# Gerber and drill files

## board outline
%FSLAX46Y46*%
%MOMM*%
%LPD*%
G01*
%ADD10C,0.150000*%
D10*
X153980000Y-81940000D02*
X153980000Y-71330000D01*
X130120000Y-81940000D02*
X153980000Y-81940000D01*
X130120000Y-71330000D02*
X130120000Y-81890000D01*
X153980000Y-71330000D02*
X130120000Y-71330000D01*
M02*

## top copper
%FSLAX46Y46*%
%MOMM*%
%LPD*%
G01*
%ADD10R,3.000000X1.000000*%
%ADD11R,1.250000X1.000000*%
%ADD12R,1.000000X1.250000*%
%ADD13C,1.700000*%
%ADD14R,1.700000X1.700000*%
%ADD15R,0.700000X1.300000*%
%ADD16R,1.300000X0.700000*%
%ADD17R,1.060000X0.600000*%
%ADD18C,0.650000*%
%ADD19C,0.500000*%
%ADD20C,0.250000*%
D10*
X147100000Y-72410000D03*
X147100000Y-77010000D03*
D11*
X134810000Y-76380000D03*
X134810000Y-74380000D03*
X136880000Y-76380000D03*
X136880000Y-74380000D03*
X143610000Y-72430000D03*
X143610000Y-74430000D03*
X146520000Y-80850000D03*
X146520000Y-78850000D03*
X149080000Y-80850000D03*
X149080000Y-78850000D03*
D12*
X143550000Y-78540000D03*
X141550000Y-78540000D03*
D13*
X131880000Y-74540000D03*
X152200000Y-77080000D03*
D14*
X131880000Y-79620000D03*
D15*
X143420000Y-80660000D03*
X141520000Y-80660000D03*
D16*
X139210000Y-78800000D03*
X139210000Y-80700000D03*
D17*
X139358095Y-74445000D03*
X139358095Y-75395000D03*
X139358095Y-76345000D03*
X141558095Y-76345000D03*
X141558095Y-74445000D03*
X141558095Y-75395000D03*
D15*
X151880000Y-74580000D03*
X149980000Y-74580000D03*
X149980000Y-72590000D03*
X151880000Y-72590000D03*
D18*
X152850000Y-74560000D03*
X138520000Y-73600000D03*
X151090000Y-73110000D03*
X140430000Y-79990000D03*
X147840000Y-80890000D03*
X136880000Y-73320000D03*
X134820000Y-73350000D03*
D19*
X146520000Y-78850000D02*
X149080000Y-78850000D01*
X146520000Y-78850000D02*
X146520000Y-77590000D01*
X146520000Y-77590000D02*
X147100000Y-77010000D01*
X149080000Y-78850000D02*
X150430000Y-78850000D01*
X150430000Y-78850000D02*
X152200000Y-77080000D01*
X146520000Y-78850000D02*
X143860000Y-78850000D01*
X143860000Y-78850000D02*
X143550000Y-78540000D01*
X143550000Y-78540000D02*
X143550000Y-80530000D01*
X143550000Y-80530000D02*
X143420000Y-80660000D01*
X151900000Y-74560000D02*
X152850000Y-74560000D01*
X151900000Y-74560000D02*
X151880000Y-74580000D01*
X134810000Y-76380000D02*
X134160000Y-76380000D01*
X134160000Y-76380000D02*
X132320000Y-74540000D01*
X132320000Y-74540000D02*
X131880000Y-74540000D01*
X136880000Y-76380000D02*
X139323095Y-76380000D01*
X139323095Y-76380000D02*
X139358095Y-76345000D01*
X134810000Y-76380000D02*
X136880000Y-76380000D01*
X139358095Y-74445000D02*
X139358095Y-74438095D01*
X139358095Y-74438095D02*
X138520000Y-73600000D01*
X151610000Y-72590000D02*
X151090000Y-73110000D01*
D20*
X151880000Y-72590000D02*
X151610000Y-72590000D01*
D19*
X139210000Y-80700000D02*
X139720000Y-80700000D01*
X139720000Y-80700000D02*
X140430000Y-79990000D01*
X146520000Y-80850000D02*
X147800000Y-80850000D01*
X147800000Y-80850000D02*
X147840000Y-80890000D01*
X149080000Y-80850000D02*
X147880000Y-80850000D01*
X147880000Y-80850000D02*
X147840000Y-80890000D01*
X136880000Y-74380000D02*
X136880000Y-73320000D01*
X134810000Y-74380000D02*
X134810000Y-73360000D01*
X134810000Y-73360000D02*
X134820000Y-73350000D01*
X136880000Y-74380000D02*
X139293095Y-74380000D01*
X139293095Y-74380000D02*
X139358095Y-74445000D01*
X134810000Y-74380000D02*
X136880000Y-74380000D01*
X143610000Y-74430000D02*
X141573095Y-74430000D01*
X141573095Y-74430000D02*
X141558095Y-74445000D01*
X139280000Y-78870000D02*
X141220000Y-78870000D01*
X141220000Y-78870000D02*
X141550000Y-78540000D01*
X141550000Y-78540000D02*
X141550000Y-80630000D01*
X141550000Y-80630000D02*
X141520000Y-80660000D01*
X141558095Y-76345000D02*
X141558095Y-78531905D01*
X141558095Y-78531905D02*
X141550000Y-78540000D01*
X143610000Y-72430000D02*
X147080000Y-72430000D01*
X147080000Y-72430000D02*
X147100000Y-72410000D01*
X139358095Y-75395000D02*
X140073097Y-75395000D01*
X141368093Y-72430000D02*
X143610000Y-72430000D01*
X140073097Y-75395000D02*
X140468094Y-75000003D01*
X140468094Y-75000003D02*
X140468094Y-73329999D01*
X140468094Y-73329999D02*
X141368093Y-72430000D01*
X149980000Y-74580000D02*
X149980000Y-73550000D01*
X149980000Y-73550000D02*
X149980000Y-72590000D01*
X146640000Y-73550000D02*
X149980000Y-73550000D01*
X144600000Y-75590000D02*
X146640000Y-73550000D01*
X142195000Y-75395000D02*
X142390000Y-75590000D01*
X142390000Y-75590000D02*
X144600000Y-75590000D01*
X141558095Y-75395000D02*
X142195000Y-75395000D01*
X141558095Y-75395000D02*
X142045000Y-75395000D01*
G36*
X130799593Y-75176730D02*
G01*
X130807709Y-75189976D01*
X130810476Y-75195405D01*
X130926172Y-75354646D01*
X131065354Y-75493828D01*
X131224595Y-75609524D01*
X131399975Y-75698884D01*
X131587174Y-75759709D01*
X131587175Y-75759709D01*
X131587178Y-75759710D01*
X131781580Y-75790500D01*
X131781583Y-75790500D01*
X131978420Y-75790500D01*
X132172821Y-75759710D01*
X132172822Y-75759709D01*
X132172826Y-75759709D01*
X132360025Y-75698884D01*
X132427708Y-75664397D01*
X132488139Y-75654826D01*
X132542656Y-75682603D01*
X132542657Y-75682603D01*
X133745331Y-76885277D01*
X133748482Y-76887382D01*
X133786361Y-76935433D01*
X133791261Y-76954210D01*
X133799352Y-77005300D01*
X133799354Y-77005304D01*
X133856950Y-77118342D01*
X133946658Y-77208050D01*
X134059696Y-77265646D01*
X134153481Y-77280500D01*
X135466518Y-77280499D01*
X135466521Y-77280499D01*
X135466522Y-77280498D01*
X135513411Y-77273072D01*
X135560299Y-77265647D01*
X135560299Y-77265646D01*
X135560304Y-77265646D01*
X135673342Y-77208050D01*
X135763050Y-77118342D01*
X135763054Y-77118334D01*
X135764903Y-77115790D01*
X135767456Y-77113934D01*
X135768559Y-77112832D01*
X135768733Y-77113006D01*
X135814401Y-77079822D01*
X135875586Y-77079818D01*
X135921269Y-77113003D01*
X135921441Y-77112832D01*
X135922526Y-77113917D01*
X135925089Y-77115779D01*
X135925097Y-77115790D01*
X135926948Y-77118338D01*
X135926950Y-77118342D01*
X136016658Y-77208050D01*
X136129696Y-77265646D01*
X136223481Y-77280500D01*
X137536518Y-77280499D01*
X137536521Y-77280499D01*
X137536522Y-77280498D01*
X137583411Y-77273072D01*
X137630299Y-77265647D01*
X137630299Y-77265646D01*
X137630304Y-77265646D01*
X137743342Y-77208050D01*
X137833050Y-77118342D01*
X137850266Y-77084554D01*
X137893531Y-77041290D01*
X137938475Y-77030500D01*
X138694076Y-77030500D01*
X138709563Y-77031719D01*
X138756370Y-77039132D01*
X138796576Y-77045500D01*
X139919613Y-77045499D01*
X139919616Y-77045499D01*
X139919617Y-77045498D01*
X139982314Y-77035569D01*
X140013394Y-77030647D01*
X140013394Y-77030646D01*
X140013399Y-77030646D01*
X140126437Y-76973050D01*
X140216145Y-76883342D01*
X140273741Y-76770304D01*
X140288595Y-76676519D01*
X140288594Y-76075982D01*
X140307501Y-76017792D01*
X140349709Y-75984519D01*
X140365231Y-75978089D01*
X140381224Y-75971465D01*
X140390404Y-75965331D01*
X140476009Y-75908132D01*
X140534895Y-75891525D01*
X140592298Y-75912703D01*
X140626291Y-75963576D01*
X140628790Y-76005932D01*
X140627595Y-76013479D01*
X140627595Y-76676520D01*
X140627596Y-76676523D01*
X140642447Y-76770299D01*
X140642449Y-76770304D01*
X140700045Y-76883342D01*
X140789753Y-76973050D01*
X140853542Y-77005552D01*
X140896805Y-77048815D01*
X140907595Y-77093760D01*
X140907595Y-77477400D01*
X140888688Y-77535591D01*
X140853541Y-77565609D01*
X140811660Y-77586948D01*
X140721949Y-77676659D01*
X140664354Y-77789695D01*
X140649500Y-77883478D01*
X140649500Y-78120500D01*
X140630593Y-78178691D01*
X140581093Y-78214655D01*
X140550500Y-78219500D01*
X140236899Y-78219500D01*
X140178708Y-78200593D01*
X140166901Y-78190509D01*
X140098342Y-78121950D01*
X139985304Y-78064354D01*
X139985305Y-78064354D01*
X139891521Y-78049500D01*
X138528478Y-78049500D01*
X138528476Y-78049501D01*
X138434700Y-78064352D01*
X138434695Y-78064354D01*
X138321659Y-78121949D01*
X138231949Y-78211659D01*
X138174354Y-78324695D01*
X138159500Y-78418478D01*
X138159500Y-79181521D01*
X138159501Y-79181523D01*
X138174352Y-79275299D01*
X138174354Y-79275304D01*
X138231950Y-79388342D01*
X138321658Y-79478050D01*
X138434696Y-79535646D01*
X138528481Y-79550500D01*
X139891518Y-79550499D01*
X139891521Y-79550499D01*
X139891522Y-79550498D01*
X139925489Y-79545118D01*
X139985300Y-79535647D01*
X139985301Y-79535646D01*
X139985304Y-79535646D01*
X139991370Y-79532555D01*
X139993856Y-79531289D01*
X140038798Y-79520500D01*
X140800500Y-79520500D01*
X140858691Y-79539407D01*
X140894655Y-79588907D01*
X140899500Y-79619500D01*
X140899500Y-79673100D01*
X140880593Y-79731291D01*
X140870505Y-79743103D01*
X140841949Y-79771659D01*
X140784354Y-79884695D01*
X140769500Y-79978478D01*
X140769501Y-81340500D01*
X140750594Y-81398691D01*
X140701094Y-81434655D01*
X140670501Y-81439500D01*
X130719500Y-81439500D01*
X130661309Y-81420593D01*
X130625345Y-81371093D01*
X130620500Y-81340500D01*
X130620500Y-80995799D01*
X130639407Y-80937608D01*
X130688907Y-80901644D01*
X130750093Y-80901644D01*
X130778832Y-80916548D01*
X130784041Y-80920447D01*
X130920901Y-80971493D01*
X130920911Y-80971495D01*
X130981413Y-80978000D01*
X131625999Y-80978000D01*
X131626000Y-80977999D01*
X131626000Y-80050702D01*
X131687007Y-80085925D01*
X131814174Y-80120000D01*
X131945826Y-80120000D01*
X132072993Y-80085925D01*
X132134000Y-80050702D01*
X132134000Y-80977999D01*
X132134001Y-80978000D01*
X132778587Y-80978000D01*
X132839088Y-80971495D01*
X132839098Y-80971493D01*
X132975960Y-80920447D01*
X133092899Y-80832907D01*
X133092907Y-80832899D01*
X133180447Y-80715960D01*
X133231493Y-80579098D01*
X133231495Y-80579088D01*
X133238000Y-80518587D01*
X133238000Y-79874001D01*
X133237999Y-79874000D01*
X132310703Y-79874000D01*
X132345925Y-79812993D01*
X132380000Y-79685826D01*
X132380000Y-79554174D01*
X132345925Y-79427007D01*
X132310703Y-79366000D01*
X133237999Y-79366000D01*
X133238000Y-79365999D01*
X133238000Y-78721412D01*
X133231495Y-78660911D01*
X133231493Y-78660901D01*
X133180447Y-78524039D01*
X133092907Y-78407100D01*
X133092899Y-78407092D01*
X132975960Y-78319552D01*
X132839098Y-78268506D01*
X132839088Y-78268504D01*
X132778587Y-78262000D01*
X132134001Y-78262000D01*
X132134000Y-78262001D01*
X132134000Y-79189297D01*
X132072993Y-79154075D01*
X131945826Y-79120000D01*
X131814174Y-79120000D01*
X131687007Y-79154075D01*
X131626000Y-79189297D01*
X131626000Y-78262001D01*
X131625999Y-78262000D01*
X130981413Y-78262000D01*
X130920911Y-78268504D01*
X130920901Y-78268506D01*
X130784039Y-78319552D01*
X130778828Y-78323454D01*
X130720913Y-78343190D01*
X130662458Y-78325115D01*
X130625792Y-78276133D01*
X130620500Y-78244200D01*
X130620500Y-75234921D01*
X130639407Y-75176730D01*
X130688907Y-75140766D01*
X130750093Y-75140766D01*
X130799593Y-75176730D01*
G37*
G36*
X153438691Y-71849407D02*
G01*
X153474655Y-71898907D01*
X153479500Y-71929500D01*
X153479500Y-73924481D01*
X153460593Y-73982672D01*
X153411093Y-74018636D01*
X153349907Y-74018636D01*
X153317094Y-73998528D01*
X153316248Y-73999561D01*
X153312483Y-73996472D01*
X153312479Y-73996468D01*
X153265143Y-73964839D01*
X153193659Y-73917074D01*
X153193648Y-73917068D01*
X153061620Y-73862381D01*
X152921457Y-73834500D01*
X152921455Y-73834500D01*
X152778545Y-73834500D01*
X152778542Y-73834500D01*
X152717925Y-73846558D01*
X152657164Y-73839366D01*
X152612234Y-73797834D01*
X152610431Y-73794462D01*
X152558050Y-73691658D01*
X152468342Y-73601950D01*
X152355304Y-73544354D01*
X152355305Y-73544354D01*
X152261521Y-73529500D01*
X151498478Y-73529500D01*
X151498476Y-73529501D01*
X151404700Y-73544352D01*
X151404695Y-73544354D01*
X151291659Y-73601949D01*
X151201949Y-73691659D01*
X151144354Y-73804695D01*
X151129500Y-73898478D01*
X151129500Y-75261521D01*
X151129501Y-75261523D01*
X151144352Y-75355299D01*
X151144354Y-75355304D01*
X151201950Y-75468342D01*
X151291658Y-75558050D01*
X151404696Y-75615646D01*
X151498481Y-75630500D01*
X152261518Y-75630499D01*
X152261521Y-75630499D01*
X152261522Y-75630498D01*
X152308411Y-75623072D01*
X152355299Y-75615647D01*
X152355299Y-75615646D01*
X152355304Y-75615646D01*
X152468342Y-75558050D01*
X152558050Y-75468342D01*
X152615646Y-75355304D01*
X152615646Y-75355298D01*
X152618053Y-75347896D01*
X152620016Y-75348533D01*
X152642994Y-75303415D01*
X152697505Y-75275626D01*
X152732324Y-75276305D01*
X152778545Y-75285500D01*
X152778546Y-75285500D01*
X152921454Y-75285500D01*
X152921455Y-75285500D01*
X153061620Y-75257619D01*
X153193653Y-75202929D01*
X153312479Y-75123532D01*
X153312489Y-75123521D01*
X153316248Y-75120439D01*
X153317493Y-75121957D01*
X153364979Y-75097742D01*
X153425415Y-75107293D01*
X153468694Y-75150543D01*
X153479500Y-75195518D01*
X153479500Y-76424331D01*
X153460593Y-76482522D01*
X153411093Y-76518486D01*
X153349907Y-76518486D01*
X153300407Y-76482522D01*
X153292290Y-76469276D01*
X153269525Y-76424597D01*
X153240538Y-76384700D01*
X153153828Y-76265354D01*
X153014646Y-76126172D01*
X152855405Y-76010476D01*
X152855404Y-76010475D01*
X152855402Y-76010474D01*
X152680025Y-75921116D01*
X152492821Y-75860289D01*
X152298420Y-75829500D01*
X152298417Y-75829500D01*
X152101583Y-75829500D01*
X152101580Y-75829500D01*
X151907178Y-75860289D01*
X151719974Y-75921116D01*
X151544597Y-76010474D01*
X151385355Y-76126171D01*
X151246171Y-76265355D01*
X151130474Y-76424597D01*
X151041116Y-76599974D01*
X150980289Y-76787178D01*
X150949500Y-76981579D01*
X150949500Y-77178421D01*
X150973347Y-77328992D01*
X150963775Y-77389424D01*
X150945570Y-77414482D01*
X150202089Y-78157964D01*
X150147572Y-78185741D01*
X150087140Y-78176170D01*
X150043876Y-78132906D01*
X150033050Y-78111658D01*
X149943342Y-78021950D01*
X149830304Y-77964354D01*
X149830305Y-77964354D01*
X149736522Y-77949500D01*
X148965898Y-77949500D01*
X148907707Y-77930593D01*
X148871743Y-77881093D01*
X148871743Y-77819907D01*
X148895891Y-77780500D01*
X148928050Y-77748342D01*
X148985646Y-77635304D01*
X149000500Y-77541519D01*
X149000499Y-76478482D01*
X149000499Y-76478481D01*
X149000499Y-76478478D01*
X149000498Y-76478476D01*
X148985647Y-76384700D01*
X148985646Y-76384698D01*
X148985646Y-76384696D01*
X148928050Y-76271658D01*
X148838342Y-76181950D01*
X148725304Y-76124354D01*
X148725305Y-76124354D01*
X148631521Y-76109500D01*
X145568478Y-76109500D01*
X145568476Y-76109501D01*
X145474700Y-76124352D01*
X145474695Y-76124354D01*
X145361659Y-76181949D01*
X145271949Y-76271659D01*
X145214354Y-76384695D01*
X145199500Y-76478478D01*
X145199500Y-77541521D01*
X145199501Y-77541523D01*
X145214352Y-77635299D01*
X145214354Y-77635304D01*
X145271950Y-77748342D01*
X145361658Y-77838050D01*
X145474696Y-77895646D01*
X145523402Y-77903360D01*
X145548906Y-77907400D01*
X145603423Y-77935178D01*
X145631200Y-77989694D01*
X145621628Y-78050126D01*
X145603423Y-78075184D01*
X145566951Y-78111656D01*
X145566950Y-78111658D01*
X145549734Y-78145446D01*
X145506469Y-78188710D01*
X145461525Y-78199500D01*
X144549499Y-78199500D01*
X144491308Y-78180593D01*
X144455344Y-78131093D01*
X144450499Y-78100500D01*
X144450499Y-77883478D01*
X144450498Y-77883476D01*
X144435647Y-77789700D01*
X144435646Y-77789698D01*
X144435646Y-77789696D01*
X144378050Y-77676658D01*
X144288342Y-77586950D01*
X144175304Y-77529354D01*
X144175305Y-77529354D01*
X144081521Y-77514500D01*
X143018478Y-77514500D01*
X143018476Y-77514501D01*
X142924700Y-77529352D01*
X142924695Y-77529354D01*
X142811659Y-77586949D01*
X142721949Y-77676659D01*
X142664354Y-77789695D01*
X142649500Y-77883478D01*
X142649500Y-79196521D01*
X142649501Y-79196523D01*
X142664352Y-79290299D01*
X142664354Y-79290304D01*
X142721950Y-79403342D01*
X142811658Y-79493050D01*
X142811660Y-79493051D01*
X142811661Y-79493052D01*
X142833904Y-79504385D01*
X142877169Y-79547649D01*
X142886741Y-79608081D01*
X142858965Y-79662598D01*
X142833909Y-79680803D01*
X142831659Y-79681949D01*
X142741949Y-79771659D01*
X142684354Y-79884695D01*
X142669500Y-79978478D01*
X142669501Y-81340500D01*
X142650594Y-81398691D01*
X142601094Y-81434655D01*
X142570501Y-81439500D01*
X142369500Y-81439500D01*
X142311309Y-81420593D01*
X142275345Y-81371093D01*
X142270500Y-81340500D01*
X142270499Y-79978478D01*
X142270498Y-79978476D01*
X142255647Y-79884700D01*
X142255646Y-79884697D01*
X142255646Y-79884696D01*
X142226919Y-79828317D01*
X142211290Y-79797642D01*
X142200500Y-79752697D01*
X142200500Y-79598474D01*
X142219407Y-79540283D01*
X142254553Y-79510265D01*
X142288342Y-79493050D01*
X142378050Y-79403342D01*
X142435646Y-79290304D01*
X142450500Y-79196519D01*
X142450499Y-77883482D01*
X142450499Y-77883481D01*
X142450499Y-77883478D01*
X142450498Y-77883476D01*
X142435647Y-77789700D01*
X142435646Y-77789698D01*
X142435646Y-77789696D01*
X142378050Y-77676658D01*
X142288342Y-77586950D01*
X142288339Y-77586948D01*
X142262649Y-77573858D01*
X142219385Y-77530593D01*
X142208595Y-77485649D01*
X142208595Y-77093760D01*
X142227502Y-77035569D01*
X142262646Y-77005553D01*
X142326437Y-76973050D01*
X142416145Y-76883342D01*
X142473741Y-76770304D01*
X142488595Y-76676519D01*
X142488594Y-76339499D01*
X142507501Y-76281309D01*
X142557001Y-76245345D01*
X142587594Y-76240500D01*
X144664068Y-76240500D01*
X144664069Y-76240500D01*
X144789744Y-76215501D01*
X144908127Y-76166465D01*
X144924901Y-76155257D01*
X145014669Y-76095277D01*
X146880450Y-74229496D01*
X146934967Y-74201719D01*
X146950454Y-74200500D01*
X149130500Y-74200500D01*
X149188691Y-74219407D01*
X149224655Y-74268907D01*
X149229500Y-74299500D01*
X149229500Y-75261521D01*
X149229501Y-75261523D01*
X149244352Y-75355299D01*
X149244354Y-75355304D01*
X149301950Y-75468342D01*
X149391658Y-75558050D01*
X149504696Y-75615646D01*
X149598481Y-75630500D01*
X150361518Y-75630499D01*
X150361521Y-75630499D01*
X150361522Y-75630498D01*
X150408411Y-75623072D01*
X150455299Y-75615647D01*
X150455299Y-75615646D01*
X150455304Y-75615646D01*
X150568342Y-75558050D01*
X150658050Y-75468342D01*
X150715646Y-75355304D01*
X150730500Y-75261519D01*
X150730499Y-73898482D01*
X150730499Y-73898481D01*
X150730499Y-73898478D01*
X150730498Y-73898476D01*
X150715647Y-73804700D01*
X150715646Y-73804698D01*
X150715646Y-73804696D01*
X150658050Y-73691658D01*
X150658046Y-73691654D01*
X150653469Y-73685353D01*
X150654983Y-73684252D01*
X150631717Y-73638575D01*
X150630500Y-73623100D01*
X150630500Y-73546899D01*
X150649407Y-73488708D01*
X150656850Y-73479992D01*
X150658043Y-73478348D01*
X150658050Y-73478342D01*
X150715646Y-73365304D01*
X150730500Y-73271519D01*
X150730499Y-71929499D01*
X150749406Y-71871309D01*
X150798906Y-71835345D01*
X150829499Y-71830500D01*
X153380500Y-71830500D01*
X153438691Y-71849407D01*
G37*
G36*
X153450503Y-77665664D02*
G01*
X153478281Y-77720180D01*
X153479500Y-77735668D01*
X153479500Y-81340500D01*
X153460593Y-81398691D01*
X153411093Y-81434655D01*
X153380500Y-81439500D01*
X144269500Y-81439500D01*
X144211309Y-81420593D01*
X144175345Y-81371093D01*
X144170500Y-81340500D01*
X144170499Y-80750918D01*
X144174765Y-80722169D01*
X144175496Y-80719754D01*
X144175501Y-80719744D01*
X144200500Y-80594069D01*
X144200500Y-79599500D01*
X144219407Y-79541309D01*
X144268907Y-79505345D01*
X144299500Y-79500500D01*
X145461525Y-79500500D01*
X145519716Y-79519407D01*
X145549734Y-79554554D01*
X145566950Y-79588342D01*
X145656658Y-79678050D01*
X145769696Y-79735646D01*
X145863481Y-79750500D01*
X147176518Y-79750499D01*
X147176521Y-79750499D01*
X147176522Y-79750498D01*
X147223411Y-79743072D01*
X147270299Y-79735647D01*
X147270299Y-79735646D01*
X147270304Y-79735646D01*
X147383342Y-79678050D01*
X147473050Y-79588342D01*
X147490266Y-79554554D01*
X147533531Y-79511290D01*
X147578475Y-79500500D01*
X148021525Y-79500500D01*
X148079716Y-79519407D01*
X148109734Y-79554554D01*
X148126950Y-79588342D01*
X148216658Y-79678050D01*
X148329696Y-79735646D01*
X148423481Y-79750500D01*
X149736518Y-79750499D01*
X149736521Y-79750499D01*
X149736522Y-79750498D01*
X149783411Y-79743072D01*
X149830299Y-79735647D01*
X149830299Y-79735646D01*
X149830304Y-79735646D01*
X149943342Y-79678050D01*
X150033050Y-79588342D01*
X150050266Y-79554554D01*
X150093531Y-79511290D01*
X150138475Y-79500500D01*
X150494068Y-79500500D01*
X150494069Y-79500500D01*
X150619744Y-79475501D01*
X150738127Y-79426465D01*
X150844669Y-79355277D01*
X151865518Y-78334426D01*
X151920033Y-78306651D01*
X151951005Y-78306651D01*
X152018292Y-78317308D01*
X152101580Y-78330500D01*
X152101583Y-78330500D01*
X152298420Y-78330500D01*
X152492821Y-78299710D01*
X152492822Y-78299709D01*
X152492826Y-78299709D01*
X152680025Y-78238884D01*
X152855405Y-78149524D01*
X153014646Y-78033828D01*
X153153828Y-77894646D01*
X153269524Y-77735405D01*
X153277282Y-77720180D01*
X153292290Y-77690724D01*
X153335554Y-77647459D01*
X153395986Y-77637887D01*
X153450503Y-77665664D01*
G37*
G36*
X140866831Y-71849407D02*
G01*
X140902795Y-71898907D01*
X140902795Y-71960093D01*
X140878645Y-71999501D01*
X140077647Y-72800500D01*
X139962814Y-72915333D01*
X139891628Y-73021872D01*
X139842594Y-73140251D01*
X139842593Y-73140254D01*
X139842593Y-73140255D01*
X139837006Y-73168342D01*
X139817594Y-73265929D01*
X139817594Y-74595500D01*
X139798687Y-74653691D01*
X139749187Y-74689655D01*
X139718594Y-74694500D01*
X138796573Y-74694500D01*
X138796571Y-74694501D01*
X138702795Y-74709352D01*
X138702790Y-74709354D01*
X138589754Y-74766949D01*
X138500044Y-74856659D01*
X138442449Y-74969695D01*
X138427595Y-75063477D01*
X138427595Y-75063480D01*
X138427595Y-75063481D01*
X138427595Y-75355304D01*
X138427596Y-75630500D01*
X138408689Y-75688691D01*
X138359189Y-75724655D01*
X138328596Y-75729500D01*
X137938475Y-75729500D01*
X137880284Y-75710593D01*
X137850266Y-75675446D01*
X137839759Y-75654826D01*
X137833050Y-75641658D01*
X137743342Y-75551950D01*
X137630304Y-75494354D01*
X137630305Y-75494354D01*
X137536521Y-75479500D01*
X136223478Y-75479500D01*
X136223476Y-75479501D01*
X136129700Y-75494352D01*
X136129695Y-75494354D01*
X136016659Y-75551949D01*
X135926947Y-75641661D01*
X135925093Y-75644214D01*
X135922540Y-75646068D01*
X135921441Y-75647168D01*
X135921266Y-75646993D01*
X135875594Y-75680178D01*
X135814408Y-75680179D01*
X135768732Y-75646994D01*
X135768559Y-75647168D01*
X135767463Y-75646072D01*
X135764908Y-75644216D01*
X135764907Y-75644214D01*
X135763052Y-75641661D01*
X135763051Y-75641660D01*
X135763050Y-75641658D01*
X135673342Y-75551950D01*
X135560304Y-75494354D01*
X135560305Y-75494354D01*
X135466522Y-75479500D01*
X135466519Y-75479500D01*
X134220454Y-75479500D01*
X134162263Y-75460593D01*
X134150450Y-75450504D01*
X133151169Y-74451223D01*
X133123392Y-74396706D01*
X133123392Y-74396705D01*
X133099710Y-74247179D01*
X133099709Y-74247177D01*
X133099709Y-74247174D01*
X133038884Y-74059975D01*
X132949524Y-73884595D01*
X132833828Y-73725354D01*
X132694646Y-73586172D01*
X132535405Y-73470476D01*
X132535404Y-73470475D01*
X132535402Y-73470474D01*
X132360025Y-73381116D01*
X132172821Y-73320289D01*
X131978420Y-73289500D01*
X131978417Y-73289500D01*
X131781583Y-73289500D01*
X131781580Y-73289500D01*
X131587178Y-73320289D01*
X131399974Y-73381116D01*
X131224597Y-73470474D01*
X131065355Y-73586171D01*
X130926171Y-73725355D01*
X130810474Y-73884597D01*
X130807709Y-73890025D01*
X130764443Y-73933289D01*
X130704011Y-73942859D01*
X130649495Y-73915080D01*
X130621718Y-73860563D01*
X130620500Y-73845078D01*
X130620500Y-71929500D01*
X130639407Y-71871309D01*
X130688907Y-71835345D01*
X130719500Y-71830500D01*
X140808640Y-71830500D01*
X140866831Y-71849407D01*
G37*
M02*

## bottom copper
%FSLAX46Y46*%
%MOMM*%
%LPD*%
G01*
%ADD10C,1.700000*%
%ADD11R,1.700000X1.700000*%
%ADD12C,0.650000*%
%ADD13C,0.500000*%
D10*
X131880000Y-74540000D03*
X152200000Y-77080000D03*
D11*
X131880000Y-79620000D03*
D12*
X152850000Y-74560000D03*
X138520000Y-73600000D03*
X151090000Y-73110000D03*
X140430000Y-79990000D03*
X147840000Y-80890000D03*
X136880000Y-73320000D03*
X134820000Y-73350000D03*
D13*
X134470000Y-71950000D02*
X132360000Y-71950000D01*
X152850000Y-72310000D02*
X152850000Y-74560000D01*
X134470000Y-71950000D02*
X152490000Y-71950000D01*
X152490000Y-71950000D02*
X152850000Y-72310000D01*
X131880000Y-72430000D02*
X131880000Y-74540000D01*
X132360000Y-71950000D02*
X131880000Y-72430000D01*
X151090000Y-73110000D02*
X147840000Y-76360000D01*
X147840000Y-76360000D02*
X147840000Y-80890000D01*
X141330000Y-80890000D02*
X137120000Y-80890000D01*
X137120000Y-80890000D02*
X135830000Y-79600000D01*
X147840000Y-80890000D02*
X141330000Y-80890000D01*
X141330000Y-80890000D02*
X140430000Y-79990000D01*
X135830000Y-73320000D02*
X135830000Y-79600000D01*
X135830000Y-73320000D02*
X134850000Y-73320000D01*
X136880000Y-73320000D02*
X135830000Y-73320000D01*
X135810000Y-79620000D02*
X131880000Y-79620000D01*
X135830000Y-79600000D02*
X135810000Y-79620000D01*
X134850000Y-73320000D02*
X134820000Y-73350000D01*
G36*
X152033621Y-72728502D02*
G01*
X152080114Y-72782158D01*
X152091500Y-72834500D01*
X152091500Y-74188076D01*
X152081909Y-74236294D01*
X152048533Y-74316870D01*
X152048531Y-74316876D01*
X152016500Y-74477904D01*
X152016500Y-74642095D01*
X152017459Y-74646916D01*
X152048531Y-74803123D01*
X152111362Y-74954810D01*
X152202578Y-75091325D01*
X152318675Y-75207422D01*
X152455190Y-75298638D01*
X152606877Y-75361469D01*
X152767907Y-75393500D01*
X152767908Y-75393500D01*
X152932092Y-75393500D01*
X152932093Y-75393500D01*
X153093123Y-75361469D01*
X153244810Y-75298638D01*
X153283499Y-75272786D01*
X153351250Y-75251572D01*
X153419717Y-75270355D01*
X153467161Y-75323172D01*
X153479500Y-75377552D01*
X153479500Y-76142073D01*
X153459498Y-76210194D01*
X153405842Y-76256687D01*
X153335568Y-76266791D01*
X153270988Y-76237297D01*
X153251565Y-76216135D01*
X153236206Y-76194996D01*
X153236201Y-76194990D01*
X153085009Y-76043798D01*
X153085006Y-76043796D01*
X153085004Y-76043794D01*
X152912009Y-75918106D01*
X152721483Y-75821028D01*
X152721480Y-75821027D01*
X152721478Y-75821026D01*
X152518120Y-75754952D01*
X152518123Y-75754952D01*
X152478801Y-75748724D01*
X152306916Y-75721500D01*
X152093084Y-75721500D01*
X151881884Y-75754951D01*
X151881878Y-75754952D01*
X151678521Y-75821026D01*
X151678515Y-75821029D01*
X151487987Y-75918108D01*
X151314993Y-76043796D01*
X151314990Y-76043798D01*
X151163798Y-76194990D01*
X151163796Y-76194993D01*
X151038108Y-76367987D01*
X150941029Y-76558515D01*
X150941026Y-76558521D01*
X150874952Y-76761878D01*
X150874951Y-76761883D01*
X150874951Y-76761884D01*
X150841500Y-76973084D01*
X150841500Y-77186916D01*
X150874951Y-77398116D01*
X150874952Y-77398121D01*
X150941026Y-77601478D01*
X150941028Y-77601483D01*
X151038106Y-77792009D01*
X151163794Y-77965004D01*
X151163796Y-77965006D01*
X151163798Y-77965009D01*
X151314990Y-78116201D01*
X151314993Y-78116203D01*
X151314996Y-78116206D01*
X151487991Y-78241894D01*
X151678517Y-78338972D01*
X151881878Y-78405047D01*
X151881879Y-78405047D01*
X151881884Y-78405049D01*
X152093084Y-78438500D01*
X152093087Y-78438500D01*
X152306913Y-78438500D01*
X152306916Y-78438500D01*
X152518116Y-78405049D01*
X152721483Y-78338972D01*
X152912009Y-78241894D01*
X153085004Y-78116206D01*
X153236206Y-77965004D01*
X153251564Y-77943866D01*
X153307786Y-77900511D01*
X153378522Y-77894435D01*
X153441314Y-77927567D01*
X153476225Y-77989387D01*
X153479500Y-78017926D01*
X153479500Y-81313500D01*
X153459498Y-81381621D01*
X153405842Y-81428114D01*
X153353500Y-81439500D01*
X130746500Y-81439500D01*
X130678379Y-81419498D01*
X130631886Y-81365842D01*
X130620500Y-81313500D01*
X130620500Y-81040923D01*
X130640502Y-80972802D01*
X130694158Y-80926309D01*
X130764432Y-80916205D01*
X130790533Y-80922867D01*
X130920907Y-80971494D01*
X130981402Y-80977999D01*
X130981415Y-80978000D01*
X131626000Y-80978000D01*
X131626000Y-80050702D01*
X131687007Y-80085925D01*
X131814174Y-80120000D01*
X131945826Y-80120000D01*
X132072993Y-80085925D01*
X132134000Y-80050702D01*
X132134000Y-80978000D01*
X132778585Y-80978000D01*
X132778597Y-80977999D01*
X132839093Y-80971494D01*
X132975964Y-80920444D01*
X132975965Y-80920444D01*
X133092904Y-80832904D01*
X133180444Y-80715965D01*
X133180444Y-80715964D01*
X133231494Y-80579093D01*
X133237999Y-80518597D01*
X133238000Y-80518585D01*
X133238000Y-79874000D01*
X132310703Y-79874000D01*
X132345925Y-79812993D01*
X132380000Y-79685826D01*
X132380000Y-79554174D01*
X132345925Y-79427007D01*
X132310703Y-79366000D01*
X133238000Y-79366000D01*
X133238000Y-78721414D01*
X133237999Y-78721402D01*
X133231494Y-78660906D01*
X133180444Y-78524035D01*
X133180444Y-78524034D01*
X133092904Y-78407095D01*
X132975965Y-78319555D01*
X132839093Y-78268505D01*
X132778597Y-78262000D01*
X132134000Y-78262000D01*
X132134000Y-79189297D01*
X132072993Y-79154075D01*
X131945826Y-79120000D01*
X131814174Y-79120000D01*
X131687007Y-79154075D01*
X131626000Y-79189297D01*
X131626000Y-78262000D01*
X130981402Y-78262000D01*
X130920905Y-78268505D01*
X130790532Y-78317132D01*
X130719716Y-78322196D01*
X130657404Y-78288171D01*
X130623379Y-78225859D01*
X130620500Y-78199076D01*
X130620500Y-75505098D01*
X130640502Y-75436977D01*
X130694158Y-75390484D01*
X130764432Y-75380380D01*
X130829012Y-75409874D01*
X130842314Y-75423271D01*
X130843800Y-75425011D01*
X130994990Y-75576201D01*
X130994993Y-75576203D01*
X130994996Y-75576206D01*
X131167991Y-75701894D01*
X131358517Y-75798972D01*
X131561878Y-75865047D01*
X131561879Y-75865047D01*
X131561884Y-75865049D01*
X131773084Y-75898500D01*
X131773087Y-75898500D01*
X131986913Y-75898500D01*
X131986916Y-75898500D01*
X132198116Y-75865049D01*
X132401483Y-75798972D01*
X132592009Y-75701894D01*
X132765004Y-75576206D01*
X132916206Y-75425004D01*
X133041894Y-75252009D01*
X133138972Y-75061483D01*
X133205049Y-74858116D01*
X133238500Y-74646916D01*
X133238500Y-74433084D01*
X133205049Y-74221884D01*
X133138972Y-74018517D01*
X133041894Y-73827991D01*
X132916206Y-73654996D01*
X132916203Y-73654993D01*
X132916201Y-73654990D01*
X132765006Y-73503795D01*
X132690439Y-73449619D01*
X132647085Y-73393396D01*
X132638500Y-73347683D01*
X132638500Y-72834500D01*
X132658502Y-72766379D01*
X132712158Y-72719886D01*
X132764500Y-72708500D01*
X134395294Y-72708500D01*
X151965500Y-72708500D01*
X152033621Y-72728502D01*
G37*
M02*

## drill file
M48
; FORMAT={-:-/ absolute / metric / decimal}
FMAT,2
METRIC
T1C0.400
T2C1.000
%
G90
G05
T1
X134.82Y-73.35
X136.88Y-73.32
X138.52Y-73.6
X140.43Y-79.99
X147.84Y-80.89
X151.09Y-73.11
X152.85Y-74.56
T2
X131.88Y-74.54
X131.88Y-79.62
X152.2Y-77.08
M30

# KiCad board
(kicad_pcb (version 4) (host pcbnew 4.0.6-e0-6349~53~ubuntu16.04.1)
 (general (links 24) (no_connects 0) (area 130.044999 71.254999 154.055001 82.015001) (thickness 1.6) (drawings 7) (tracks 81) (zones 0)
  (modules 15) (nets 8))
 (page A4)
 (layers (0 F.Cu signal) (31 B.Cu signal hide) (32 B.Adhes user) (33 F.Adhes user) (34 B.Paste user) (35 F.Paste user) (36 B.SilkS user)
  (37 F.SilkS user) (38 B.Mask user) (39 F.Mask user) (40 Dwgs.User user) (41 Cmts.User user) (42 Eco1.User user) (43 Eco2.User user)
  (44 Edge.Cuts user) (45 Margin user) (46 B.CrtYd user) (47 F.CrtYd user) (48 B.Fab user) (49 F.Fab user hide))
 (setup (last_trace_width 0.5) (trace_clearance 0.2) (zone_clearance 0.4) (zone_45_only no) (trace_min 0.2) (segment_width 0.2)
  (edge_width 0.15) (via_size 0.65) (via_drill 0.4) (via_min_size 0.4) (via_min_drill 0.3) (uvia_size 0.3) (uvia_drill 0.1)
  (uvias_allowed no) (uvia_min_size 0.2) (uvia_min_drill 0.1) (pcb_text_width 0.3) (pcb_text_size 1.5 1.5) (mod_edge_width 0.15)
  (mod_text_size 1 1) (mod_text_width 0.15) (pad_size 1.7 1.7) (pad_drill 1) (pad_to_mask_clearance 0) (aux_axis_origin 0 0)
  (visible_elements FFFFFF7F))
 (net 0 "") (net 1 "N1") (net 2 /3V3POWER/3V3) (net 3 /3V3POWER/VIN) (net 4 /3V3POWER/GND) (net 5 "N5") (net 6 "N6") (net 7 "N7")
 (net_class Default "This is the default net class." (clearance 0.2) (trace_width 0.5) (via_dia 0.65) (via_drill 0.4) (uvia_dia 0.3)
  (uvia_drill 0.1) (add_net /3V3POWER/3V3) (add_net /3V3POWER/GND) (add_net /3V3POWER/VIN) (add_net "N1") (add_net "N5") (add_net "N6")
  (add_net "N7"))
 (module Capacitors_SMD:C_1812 (layer F.Cu) (at 147.1 74.71 270)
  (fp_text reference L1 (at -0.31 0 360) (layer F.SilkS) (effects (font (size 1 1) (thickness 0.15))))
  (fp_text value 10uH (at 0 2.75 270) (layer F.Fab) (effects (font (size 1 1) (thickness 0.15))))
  (pad 1 smd rect (at -2.3 0 270) (size 1 3) (layers F.Cu F.Paste F.Mask) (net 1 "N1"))
  (pad 2 smd rect (at 2.3 0 270) (size 1 3) (layers F.Cu F.Paste F.Mask) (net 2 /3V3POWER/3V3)))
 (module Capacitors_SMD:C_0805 (layer F.Cu) (at 134.81 75.38 90)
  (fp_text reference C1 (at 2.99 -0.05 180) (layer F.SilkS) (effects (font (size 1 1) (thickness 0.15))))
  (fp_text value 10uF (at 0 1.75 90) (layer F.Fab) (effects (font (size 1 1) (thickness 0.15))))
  (pad 1 smd rect (at -1 0 90) (size 1 1.25) (layers F.Cu F.Paste F.Mask) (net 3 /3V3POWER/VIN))
  (pad 2 smd rect (at 1 0 90) (size 1 1.25) (layers F.Cu F.Paste F.Mask) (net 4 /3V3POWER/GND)))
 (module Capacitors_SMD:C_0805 (layer F.Cu) (at 136.88 75.38 90)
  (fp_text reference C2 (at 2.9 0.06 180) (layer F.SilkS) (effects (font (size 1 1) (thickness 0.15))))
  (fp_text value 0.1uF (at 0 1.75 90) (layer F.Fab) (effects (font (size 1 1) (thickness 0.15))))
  (pad 1 smd rect (at -1 0 90) (size 1 1.25) (layers F.Cu F.Paste F.Mask) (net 3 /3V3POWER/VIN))
  (pad 2 smd rect (at 1 0 90) (size 1 1.25) (layers F.Cu F.Paste F.Mask) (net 4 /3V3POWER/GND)))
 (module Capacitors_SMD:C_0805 (layer F.Cu) (at 143.61 73.43 270)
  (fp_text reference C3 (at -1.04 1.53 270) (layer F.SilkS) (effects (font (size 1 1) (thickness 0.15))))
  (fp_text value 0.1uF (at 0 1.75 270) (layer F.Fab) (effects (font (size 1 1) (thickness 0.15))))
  (pad 1 smd rect (at -1 0 270) (size 1 1.25) (layers F.Cu F.Paste F.Mask) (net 1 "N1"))
  (pad 2 smd rect (at 1 0 270) (size 1 1.25) (layers F.Cu F.Paste F.Mask) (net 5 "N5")))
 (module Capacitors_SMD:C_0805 (layer F.Cu) (at 146.52 79.85 90)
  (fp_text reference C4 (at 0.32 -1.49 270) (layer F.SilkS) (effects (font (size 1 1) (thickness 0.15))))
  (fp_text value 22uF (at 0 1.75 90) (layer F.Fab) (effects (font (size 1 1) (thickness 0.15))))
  (pad 1 smd rect (at -1 0 90) (size 1 1.25) (layers F.Cu F.Paste F.Mask) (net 4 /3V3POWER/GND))
  (pad 2 smd rect (at 1 0 90) (size 1 1.25) (layers F.Cu F.Paste F.Mask) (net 2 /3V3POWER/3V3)))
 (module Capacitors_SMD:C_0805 (layer F.Cu) (at 149.08 79.85 90)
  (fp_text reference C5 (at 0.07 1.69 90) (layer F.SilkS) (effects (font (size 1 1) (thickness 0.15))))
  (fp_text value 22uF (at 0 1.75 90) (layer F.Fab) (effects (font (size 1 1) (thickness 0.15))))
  (pad 1 smd rect (at -1 0 90) (size 1 1.25) (layers F.Cu F.Paste F.Mask) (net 4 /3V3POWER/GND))
  (pad 2 smd rect (at 1 0 90) (size 1 1.25) (layers F.Cu F.Paste F.Mask) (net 2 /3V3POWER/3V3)))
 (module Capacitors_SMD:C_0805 (layer F.Cu) (at 142.55 78.54 180)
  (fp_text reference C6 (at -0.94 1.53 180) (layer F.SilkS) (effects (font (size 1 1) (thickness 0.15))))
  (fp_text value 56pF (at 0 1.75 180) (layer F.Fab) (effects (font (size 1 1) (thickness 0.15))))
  (pad 1 smd rect (at -1 0 180) (size 1 1.25) (layers F.Cu F.Paste F.Mask) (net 2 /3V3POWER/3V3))
  (pad 2 smd rect (at 1 0 180) (size 1 1.25) (layers F.Cu F.Paste F.Mask) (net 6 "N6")))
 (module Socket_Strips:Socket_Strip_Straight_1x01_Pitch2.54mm (layer F.Cu) (at 131.88 74.54)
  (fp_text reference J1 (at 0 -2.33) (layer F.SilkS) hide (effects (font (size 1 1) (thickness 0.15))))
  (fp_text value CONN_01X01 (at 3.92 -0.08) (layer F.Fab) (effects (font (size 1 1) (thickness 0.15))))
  (pad 1 thru_hole circle (at 0 0) (size 1.7 1.7) (drill 1) (layers *.Cu *.Mask) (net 3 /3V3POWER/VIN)))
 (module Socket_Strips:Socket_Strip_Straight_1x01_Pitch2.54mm (layer F.Cu) (at 152.2 77.08)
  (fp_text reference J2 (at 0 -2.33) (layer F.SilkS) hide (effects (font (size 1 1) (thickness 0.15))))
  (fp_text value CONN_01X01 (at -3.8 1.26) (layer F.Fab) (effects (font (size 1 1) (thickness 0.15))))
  (pad 1 thru_hole circle (at 0 0) (size 1.7 1.7) (drill 1) (layers *.Cu *.Mask) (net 2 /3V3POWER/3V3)))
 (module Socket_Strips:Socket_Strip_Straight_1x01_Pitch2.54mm (layer F.Cu) (at 131.88 79.62)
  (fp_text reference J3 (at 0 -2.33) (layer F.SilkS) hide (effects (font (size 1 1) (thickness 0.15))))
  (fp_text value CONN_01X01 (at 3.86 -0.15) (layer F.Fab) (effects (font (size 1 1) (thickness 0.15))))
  (pad 1 thru_hole rect (at 0 0) (size 1.7 1.7) (drill 1) (layers *.Cu *.Mask) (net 4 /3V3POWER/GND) (zone_connect 1)))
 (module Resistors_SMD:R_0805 (layer F.Cu) (at 142.47 80.66 180)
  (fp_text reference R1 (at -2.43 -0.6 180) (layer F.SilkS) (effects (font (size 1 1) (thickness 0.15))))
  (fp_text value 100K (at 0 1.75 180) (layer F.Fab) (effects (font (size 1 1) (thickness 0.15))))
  (pad 1 smd rect (at -0.95 0 180) (size 0.7 1.3) (layers F.Cu F.Paste F.Mask) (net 2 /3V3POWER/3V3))
  (pad 2 smd rect (at 0.95 0 180) (size 0.7 1.3) (layers F.Cu F.Paste F.Mask) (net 6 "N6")))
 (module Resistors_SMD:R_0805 (layer F.Cu) (at 139.21 79.75 270)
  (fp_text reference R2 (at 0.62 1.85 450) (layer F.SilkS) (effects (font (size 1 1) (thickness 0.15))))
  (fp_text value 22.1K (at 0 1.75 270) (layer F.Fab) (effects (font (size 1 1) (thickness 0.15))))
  (pad 1 smd rect (at -0.95 0 270) (size 0.7 1.3) (layers F.Cu F.Paste F.Mask) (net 6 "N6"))
  (pad 2 smd rect (at 0.95 0 270) (size 0.7 1.3) (layers F.Cu F.Paste F.Mask) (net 4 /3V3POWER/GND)))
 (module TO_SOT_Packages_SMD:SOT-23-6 (layer F.Cu) (at 140.458095 75.395)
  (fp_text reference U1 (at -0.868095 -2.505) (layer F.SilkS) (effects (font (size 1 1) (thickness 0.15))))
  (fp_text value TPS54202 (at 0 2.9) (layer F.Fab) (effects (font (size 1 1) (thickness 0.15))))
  (pad 1 smd rect (at -1.1 -0.95) (size 1.06 0.6) (layers F.Cu F.Paste F.Mask) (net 4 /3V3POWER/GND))
  (pad 2 smd rect (at -1.1 0) (size 1.06 0.6) (layers F.Cu F.Paste F.Mask) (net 1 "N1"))
  (pad 3 smd rect (at -1.1 0.95) (size 1.06 0.6) (layers F.Cu F.Paste F.Mask) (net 3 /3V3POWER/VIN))
  (pad 4 smd rect (at 1.1 0.95) (size 1.06 0.6) (layers F.Cu F.Paste F.Mask) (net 6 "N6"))
  (pad 6 smd rect (at 1.1 -0.95) (size 1.06 0.6) (layers F.Cu F.Paste F.Mask) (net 5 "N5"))
  (pad 5 smd rect (at 1.1 0) (size 1.06 0.6) (layers F.Cu F.Paste F.Mask) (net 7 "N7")))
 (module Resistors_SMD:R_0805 (layer F.Cu) (at 150.93 74.58 180)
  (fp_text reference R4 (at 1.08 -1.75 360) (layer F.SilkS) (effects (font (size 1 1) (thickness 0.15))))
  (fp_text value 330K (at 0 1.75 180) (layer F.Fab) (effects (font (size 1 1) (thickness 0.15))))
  (pad 1 smd rect (at -0.95 0 180) (size 0.7 1.3) (layers F.Cu F.Paste F.Mask) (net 3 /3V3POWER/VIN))
  (pad 2 smd rect (at 0.95 0 180) (size 0.7 1.3) (layers F.Cu F.Paste F.Mask) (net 7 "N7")))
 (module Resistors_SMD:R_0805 (layer F.Cu) (at 150.93 72.59)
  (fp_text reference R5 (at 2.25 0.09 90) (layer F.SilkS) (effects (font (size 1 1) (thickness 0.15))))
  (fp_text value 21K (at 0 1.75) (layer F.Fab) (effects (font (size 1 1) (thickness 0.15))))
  (pad 1 smd rect (at -0.95 0) (size 0.7 1.3) (layers F.Cu F.Paste F.Mask) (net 7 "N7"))
  (pad 2 smd rect (at 0.95 0) (size 0.7 1.3) (layers F.Cu F.Paste F.Mask) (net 4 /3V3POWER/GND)))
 (gr_line (start 153.98 81.94) (end 153.98 71.33) (angle 90) (layer Edge.Cuts) (width 0.15))
 (gr_line (start 130.12 81.94) (end 153.98 81.94) (angle 90) (layer Edge.Cuts) (width 0.15))
 (gr_line (start 130.12 71.33) (end 130.12 81.89) (angle 90) (layer Edge.Cuts) (width 0.15))
 (gr_line (start 153.98 71.33) (end 130.12 71.33) (angle 90) (layer Edge.Cuts) (width 0.15))
 (segment (start 146.52 78.85) (end 149.08 78.85) (width 0.5) (layer F.Cu) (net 2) (status 30))
 (segment (start 146.52 78.85) (end 146.52 77.59) (width 0.5) (layer F.Cu) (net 2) (status 10))
 (segment (start 146.52 77.59) (end 147.1 77.01) (width 0.5) (layer F.Cu) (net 2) (status 20))
 (segment (start 149.08 78.85) (end 150.43 78.85) (width 0.5) (layer F.Cu) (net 2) (status 10))
 (segment (start 150.43 78.85) (end 152.2 77.08) (width 0.5) (layer F.Cu) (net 2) (status 20))
 (segment (start 146.52 78.85) (end 143.86 78.85) (width 0.5) (layer F.Cu) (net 2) (status 30))
 (segment (start 143.86 78.85) (end 143.55 78.54) (width 0.5) (layer F.Cu) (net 2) (status 30))
 (segment (start 143.55 78.54) (end 143.55 80.53) (width 0.5) (layer F.Cu) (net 2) (status 30))
 (segment (start 143.55 80.53) (end 143.42 80.66) (width 0.5) (layer F.Cu) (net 2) (status 30))
 (segment (start 134.47 71.95) (end 132.36 71.95) (width 0.5) (layer B.Cu) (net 3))
 (segment (start 152.85 72.31) (end 152.85 74.56) (width 0.5) (layer B.Cu) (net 3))
 (segment (start 151.9 74.56) (end 152.85 74.56) (width 0.5) (layer F.Cu) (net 3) (status 20))
 (segment (start 134.47 71.95) (end 152.49 71.95) (width 0.5) (layer B.Cu) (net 3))
 (via (at 152.85 74.56) (size 0.65) (drill 0.4) (layers F.Cu B.Cu) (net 3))
 (segment (start 152.49 71.95) (end 152.85 72.31) (width 0.5) (layer B.Cu) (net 3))
 (segment (start 131.88 72.43) (end 131.88 74.54) (width 0.5) (layer B.Cu) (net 3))
 (segment (start 132.36 71.95) (end 131.88 72.43) (width 0.5) (layer B.Cu) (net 3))
 (segment (start 151.9 74.56) (end 151.88 74.58) (width 0.5) (layer F.Cu) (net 3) (status 30))
 (segment (start 134.81 76.38) (end 134.16 76.38) (width 0.5) (layer F.Cu) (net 3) (status 10))
 (segment (start 134.16 76.38) (end 132.32 74.54) (width 0.5) (layer F.Cu) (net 3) (status 20))
 (segment (start 132.32 74.54) (end 131.88 74.54) (width 0.5) (layer F.Cu) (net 3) (status 30))
 (segment (start 136.88 76.38) (end 139.323095 76.38) (width 0.5) (layer F.Cu) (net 3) (status 30))
 (segment (start 139.323095 76.38) (end 139.358095 76.345) (width 0.5) (layer F.Cu) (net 3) (status 30))
 (segment (start 134.81 76.38) (end 136.88 76.38) (width 0.5) (layer F.Cu) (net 3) (status 30))
 (segment (start 139.358095 74.445) (end 139.358095 74.438095) (width 0.5) (layer F.Cu) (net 4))
 (segment (start 139.358095 74.438095) (end 138.52 73.6) (width 0.5) (layer F.Cu) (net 4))
 (via (at 138.52 73.6) (size 0.65) (drill 0.4) (layers F.Cu B.Cu) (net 4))
 (segment (start 151.09 73.11) (end 147.84 76.36) (width 0.5) (layer B.Cu) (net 4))
 (via (at 151.09 73.11) (size 0.65) (drill 0.4) (layers F.Cu B.Cu) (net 4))
 (segment (start 151.61 72.59) (end 151.09 73.11) (width 0.5) (layer F.Cu) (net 4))
 (segment (start 147.84 76.36) (end 147.84 80.89) (width 0.5) (layer B.Cu) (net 4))
 (segment (start 151.88 72.59) (end 151.61 72.59) (width 0.25) (layer F.Cu) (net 4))
 (segment (start 141.33 80.89) (end 137.12 80.89) (width 0.5) (layer B.Cu) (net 4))
 (segment (start 137.12 80.89) (end 135.83 79.6) (width 0.5) (layer B.Cu) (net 4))
 (segment (start 147.84 80.89) (end 141.33 80.89) (width 0.5) (layer B.Cu) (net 4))
 (segment (start 141.33 80.89) (end 140.43 79.99) (width 0.5) (layer B.Cu) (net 4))
 (segment (start 139.21 80.7) (end 139.72 80.7) (width 0.5) (layer F.Cu) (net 4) (status 30))
 (segment (start 139.72 80.7) (end 140.43 79.99) (width 0.5) (layer F.Cu) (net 4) (status 10))
 (via (at 140.43 79.99) (size 0.65) (drill 0.4) (layers F.Cu B.Cu) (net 4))
 (segment (start 135.83 73.32) (end 135.83 79.6) (width 0.5) (layer B.Cu) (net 4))
 (segment (start 135.83 73.32) (end 134.85 73.32) (width 0.5) (layer B.Cu) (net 4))
 (segment (start 136.88 73.32) (end 135.83 73.32) (width 0.5) (layer B.Cu) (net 4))
 (segment (start 135.81 79.62) (end 131.88 79.62) (width 0.5) (layer B.Cu) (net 4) (status 20))
 (segment (start 135.83 79.6) (end 135.81 79.62) (width 0.5) (layer B.Cu) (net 4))
 (segment (start 146.52 80.85) (end 147.8 80.85) (width 0.5) (layer F.Cu) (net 4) (status 10))
 (segment (start 147.8 80.85) (end 147.84 80.89) (width 0.5) (layer F.Cu) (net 4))
 (segment (start 149.08 80.85) (end 147.88 80.85) (width 0.5) (layer F.Cu) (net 4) (status 10))
 (segment (start 147.88 80.85) (end 147.84 80.89) (width 0.5) (layer F.Cu) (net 4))
 (via (at 147.84 80.89) (size 0.65) (drill 0.4) (layers F.Cu B.Cu) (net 4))
 (segment (start 134.85 73.32) (end 134.82 73.35) (width 0.5) (layer B.Cu) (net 4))
 (segment (start 136.88 74.38) (end 136.88 73.32) (width 0.5) (layer F.Cu) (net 4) (status 10))
 (via (at 136.88 73.32) (size 0.65) (drill 0.4) (layers F.Cu B.Cu) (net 4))
 (segment (start 134.81 74.38) (end 134.81 73.36) (width 0.5) (layer F.Cu) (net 4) (status 10))
 (segment (start 134.81 73.36) (end 134.82 73.35) (width 0.5) (layer F.Cu) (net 4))
 (via (at 134.82 73.35) (size 0.65) (drill 0.4) (layers F.Cu B.Cu) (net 4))
 (segment (start 136.88 74.38) (end 139.293095 74.38) (width 0.5) (layer F.Cu) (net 4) (status 30))
 (segment (start 139.293095 74.38) (end 139.358095 74.445) (width 0.5) (layer F.Cu) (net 4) (status 30))
 (segment (start 134.81 74.38) (end 136.88 74.38) (width 0.5) (layer F.Cu) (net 4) (status 30))
 (segment (start 143.61 74.43) (end 141.573095 74.43) (width 0.5) (layer F.Cu) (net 5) (status 30))
 (segment (start 141.573095 74.43) (end 141.558095 74.445) (width 0.5) (layer F.Cu) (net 5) (status 30))
 (segment (start 139.28 78.87) (end 141.22 78.87) (width 0.5) (layer F.Cu) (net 6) (status 30))
 (segment (start 141.22 78.87) (end 141.55 78.54) (width 0.5) (layer F.Cu) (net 6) (status 30))
 (segment (start 141.55 78.54) (end 141.55 80.63) (width 0.5) (layer F.Cu) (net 6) (status 30))
 (segment (start 141.55 80.63) (end 141.52 80.66) (width 0.5) (layer F.Cu) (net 6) (status 30))
 (segment (start 141.558095 76.345) (end 141.558095 78.531905) (width 0.5) (layer F.Cu) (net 6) (status 30))
 (segment (start 141.558095 78.531905) (end 141.55 78.54) (width 0.5) (layer F.Cu) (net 6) (status 30))
 (segment (start 143.61 72.43) (end 147.08 72.43) (width 0.5) (layer F.Cu) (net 1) (status 30))
 (segment (start 147.08 72.43) (end 147.1 72.41) (width 0.5) (layer F.Cu) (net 1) (status 30))
 (segment (start 139.358095 75.395) (end 140.073097 75.395) (width 0.5) (layer F.Cu) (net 1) (status 10))
 (segment (start 141.368093 72.43) (end 143.61 72.43) (width 0.5) (layer F.Cu) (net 1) (status 20))
 (segment (start 140.073097 75.395) (end 140.468094 75.000003) (width 0.5) (layer F.Cu) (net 1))
 (segment (start 140.468094 75.000003) (end 140.468094 73.329999) (width 0.5) (layer F.Cu) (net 1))
 (segment (start 140.468094 73.329999) (end 141.368093 72.43) (width 0.5) (layer F.Cu) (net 1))
 (segment (start 149.98 74.58) (end 149.98 73.55) (width 0.5) (layer F.Cu) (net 7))
 (segment (start 149.98 73.55) (end 149.98 72.59) (width 0.5) (layer F.Cu) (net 7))
 (segment (start 146.64 73.55) (end 149.98 73.55) (width 0.5) (layer F.Cu) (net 7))
 (segment (start 144.6 75.59) (end 146.64 73.55) (width 0.5) (layer F.Cu) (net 7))
 (segment (start 142.195 75.395) (end 142.39 75.59) (width 0.5) (layer F.Cu) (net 7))
 (segment (start 142.39 75.59) (end 144.6 75.59) (width 0.5) (layer F.Cu) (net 7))
 (segment (start 141.558095 75.395) (end 142.195 75.395) (width 0.5) (layer F.Cu) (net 7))
 (segment (start 141.558095 75.395) (end 142.045 75.395) (width 0.5) (layer F.Cu) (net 7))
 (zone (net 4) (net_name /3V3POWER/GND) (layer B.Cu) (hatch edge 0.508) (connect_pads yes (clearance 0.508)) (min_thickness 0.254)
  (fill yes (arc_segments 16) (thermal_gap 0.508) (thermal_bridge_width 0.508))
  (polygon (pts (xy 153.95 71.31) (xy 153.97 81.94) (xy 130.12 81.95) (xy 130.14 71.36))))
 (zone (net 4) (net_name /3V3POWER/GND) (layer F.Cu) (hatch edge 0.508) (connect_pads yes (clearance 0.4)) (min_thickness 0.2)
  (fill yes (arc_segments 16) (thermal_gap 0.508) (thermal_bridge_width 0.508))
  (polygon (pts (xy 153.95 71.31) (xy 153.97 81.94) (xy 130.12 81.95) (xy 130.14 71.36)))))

